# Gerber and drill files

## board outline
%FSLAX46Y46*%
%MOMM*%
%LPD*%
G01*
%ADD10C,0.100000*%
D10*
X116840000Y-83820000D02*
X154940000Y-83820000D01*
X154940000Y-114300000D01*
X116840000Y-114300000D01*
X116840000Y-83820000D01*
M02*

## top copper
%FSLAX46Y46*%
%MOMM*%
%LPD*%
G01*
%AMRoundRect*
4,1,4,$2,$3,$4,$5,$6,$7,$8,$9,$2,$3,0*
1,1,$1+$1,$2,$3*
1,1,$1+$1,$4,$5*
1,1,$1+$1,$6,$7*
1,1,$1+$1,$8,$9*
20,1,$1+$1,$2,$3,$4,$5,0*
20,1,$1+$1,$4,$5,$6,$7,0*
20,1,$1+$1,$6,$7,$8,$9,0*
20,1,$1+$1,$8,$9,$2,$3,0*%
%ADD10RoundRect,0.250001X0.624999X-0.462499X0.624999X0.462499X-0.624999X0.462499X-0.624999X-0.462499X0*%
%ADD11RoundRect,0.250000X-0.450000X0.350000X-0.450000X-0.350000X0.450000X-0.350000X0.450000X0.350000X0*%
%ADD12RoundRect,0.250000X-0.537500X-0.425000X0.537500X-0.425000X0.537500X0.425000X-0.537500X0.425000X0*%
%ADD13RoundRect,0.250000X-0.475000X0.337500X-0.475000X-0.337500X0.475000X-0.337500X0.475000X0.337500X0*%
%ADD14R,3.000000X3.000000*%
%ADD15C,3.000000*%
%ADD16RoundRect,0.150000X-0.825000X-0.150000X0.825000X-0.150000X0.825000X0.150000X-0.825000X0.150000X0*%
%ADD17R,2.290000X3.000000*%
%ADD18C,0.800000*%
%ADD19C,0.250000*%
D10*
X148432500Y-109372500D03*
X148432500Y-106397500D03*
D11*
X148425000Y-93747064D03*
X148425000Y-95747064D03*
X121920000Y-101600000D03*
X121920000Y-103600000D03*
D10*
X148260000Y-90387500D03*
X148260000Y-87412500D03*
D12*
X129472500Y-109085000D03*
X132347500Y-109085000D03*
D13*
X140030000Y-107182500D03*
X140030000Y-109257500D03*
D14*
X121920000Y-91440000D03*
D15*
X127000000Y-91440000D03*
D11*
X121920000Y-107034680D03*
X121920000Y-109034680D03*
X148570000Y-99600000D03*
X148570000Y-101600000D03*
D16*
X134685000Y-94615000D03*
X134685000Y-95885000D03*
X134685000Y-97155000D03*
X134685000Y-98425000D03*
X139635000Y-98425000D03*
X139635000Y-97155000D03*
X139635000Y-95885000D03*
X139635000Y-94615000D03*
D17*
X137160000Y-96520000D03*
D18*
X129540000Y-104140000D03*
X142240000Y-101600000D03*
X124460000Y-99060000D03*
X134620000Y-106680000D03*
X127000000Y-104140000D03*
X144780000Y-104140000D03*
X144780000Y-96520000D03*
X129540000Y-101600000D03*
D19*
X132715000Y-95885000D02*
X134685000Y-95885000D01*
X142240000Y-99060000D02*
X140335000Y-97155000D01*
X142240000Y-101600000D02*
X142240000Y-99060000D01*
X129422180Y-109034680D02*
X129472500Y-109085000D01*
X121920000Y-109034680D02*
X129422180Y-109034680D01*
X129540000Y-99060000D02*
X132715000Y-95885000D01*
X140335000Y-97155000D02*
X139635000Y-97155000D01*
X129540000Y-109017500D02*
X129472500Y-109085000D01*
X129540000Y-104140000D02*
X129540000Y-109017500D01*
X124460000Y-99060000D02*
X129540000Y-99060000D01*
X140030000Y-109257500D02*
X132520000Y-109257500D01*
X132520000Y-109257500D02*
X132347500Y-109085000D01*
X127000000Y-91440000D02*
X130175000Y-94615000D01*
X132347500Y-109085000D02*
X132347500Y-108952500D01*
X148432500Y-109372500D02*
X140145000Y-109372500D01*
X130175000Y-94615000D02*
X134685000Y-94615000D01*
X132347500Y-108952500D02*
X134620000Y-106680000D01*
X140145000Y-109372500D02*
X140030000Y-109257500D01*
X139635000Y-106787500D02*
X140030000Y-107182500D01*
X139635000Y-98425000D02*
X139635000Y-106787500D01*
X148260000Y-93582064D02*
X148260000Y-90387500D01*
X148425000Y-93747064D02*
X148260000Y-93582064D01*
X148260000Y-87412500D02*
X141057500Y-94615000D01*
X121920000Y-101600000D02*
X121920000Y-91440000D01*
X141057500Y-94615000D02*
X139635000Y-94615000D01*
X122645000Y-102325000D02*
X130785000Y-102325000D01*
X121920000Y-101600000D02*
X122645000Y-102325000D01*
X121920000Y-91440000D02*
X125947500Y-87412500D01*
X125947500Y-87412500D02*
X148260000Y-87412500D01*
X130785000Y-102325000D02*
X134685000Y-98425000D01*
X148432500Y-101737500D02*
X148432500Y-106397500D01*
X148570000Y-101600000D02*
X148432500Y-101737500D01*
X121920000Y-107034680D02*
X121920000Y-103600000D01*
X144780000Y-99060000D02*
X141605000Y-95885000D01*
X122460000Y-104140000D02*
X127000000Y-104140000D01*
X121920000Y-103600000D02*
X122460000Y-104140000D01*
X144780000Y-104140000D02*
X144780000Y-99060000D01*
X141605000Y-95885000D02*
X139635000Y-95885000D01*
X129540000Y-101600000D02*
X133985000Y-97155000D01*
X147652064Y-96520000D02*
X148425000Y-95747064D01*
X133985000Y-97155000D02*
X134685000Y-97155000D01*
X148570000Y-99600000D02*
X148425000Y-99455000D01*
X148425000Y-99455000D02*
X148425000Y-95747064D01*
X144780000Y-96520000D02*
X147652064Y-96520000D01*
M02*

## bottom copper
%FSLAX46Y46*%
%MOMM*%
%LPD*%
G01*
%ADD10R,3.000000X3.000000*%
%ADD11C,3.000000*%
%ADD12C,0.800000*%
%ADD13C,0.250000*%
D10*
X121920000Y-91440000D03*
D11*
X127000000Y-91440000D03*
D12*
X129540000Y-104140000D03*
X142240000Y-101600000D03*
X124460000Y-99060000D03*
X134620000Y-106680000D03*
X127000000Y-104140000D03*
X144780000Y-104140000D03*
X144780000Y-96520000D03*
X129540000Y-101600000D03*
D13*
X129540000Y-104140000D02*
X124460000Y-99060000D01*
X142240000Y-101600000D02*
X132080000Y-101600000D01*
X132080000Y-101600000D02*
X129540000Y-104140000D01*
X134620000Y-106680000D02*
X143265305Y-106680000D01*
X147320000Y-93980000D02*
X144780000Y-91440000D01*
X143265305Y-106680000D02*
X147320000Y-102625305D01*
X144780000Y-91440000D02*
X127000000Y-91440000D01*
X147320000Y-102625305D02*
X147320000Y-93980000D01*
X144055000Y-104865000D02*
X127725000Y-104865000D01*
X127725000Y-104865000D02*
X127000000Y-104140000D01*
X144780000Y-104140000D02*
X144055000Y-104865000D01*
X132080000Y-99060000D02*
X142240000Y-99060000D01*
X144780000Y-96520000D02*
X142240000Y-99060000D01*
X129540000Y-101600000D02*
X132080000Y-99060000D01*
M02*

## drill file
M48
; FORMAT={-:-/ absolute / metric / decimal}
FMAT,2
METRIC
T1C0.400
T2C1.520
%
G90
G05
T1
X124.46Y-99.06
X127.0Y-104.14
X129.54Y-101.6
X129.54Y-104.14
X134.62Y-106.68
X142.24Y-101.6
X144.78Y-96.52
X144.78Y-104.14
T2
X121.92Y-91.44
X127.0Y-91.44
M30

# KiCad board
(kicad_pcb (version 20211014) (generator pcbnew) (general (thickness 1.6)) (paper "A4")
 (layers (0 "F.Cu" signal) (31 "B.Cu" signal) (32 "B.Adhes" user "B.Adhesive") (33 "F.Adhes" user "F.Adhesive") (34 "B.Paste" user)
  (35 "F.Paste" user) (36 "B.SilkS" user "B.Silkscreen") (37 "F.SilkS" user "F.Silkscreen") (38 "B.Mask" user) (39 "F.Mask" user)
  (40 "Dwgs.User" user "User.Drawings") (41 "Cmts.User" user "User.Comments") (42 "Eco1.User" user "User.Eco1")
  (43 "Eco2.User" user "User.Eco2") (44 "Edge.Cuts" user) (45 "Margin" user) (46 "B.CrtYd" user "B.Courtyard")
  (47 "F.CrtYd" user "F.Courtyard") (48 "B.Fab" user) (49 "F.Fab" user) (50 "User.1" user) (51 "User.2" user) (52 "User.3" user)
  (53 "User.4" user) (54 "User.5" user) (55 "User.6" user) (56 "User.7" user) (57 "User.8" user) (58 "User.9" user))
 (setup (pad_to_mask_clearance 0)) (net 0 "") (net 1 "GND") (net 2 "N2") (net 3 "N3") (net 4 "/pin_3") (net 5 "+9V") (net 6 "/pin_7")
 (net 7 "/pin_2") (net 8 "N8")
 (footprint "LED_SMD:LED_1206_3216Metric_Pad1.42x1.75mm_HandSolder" (layer "F.Cu") (at 148.4325 107.885 90)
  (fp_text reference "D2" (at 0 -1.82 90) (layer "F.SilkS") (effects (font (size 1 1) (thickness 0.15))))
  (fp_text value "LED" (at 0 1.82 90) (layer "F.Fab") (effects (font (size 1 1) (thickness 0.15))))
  (pad "1" smd roundrect (at -1.4875 0 90) (size 1.425 1.75) (layers "F.Cu" "F.Paste" "F.Mask") (roundrect_rratio 0.175439) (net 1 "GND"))
  (pad "2" smd roundrect (at 1.4875 0 90) (size 1.425 1.75) (layers "F.Cu" "F.Paste" "F.Mask") (roundrect_rratio 0.175439) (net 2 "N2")))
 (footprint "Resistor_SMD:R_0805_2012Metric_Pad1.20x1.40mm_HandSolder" (layer "F.Cu") (at 148.425 94.747064 -90)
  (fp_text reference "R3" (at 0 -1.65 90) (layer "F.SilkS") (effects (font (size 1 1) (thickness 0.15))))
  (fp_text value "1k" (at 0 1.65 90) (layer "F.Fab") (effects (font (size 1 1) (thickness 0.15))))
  (pad "1" smd roundrect (at -1 0 270) (size 1.2 1.4) (layers "F.Cu" "F.Paste" "F.Mask") (roundrect_rratio 0.208333) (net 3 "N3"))
  (pad "2" smd roundrect (at 1 0 270) (size 1.2 1.4) (layers "F.Cu" "F.Paste" "F.Mask") (roundrect_rratio 0.208333) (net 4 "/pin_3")))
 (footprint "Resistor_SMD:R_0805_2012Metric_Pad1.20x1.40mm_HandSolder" (layer "F.Cu") (at 121.92 102.6 -90)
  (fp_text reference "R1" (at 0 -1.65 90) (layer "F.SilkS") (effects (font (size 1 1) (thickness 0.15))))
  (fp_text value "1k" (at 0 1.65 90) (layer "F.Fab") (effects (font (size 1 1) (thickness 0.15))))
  (pad "1" smd roundrect (at -1 0 270) (size 1.2 1.4) (layers "F.Cu" "F.Paste" "F.Mask") (roundrect_rratio 0.208333) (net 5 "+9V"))
  (pad "2" smd roundrect (at 1 0 270) (size 1.2 1.4) (layers "F.Cu" "F.Paste" "F.Mask") (roundrect_rratio 0.208333) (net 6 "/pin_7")))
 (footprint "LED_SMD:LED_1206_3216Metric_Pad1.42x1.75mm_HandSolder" (layer "F.Cu") (at 148.26 88.9 90)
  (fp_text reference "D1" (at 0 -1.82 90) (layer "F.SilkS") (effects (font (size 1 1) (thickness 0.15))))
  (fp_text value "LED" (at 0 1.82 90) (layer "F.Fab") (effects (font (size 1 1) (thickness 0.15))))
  (pad "1" smd roundrect (at -1.4875 0 90) (size 1.425 1.75) (layers "F.Cu" "F.Paste" "F.Mask") (roundrect_rratio 0.175439) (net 3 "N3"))
  (pad "2" smd roundrect (at 1.4875 0 90) (size 1.425 1.75) (layers "F.Cu" "F.Paste" "F.Mask") (roundrect_rratio 0.175439) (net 5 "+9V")))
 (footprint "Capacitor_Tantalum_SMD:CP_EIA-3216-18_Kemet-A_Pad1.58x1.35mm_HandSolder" (layer "F.Cu") (at 130.91 109.085)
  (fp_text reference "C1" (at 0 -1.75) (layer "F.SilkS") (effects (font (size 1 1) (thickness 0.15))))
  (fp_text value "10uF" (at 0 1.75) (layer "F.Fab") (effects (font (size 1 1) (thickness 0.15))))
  (pad "1" smd roundrect (at -1.4375 0) (size 1.575 1.35) (layers "F.Cu" "F.Paste" "F.Mask") (roundrect_rratio 0.185185) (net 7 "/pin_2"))
  (pad "2" smd roundrect (at 1.4375 0) (size 1.575 1.35) (layers "F.Cu" "F.Paste" "F.Mask") (roundrect_rratio 0.185185) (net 1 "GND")))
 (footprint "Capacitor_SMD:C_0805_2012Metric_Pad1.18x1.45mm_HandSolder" (layer "F.Cu") (at 140.03 108.22 -90)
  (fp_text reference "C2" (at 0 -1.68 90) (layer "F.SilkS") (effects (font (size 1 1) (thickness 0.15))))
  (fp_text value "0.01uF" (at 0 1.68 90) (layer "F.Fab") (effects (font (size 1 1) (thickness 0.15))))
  (pad "1" smd roundrect (at -1.0375 0 270) (size 1.175 1.45) (layers "F.Cu" "F.Paste" "F.Mask") (roundrect_rratio 0.212766) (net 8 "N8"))
  (pad "2" smd roundrect (at 1.0375 0 270) (size 1.175 1.45) (layers "F.Cu" "F.Paste" "F.Mask") (roundrect_rratio 0.212766) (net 1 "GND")))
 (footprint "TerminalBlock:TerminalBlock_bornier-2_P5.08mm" (layer "F.Cu") (at 121.92 91.44)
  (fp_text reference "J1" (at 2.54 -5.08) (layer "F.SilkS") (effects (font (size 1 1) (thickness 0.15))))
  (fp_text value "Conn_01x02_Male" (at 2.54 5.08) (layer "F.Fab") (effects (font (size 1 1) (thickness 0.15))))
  (pad "1" thru_hole rect (at 0 0) (size 3 3) (drill 1.52) (layers *.Cu *.Mask) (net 5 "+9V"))
  (pad "2" thru_hole circle (at 5.08 0) (size 3 3) (drill 1.52) (layers *.Cu *.Mask) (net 1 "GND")))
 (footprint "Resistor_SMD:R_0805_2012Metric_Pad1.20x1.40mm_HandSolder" (layer "F.Cu") (at 121.92 108.03468 -90)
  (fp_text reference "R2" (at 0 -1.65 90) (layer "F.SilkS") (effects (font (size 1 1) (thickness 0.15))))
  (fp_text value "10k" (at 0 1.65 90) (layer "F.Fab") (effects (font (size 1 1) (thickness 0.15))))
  (pad "1" smd roundrect (at -1 0 270) (size 1.2 1.4) (layers "F.Cu" "F.Paste" "F.Mask") (roundrect_rratio 0.208333) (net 6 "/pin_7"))
  (pad "2" smd roundrect (at 1 0 270) (size 1.2 1.4) (layers "F.Cu" "F.Paste" "F.Mask") (roundrect_rratio 0.208333) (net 7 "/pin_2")))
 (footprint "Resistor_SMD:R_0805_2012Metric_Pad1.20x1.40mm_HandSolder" (layer "F.Cu") (at 148.57 100.6 -90)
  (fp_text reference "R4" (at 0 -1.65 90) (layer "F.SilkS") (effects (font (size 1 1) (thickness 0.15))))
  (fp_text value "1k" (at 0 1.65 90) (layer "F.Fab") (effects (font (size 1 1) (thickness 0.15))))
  (pad "1" smd roundrect (at -1 0 270) (size 1.2 1.4) (layers "F.Cu" "F.Paste" "F.Mask") (roundrect_rratio 0.208333) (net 4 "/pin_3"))
  (pad "2" smd roundrect (at 1 0 270) (size 1.2 1.4) (layers "F.Cu" "F.Paste" "F.Mask") (roundrect_rratio 0.208333) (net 2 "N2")))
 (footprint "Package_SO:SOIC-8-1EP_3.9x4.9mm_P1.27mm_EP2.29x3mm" (layer "F.Cu") (at 137.16 96.52)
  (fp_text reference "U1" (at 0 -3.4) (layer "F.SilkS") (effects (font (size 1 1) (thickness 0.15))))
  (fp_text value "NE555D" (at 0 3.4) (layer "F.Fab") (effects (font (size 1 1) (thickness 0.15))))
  (pad "" smd roundrect (at -0.57 0.75) (size 0.92 1.21) (layers "F.Paste") (roundrect_rratio 0.25))
  (pad "" smd roundrect (at 0.57 -0.75) (size 0.92 1.21) (layers "F.Paste") (roundrect_rratio 0.25))
  (pad "" smd roundrect (at 0.57 0.75) (size 0.92 1.21) (layers "F.Paste") (roundrect_rratio 0.25))
  (pad "" smd roundrect (at -0.57 -0.75) (size 0.92 1.21) (layers "F.Paste") (roundrect_rratio 0.25))
  (pad "1" smd roundrect (at -2.475 -1.905) (size 1.95 0.6) (layers "F.Cu" "F.Paste" "F.Mask") (roundrect_rratio 0.25) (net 1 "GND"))
  (pad "2" smd roundrect (at -2.475 -0.635) (size 1.95 0.6) (layers "F.Cu" "F.Paste" "F.Mask") (roundrect_rratio 0.25) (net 7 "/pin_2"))
  (pad "3" smd roundrect (at -2.475 0.635) (size 1.95 0.6) (layers "F.Cu" "F.Paste" "F.Mask") (roundrect_rratio 0.25) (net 4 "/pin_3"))
  (pad "4" smd roundrect (at -2.475 1.905) (size 1.95 0.6) (layers "F.Cu" "F.Paste" "F.Mask") (roundrect_rratio 0.25) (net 5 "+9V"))
  (pad "5" smd roundrect (at 2.475 1.905) (size 1.95 0.6) (layers "F.Cu" "F.Paste" "F.Mask") (roundrect_rratio 0.25) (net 8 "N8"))
  (pad "6" smd roundrect (at 2.475 0.635) (size 1.95 0.6) (layers "F.Cu" "F.Paste" "F.Mask") (roundrect_rratio 0.25) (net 7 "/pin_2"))
  (pad "7" smd roundrect (at 2.475 -0.635) (size 1.95 0.6) (layers "F.Cu" "F.Paste" "F.Mask") (roundrect_rratio 0.25) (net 6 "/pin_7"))
  (pad "8" smd roundrect (at 2.475 -1.905) (size 1.95 0.6) (layers "F.Cu" "F.Paste" "F.Mask") (roundrect_rratio 0.25) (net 5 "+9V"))
  (pad "9" smd rect (at 0 0) (size 2.29 3) (layers "F.Cu" "F.Mask")))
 (gr_rect (start 116.84 83.82) (end 154.94 114.3) (layer "Edge.Cuts") (width 0.1) (fill none))
 (segment (start 132.715 95.885) (end 134.685 95.885) (width 0.25) (layer "F.Cu") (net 7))
 (segment (start 142.24 99.06) (end 140.335 97.155) (width 0.25) (layer "F.Cu") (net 7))
 (segment (start 142.24 101.6) (end 142.24 99.06) (width 0.25) (layer "F.Cu") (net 7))
 (segment (start 129.42218 109.03468) (end 129.4725 109.085) (width 0.25) (layer "F.Cu") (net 7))
 (segment (start 121.92 109.03468) (end 129.42218 109.03468) (width 0.25) (layer "F.Cu") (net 7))
 (segment (start 129.54 99.06) (end 132.715 95.885) (width 0.25) (layer "F.Cu") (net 7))
 (segment (start 140.335 97.155) (end 139.635 97.155) (width 0.25) (layer "F.Cu") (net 7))
 (segment (start 129.54 109.0175) (end 129.4725 109.085) (width 0.25) (layer "F.Cu") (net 7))
 (segment (start 129.54 104.14) (end 129.54 109.0175) (width 0.25) (layer "F.Cu") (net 7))
 (segment (start 124.46 99.06) (end 129.54 99.06) (width 0.25) (layer "F.Cu") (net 7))
 (via (at 129.54 104.14) (size 0.8) (drill 0.4) (layers "F.Cu" "B.Cu") (free) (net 7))
 (via (at 142.24 101.6) (size 0.8) (drill 0.4) (layers "F.Cu" "B.Cu") (free) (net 7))
 (via (at 124.46 99.06) (size 0.8) (drill 0.4) (layers "F.Cu" "B.Cu") (free) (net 7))
 (segment (start 129.54 104.14) (end 124.46 99.06) (width 0.25) (layer "B.Cu") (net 7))
 (segment (start 142.24 101.6) (end 132.08 101.6) (width 0.25) (layer "B.Cu") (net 7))
 (segment (start 132.08 101.6) (end 129.54 104.14) (width 0.25) (layer "B.Cu") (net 7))
 (segment (start 140.03 109.2575) (end 132.52 109.2575) (width 0.25) (layer "F.Cu") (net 1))
 (segment (start 132.52 109.2575) (end 132.3475 109.085) (width 0.25) (layer "F.Cu") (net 1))
 (segment (start 127 91.44) (end 130.175 94.615) (width 0.25) (layer "F.Cu") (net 1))
 (segment (start 132.3475 109.085) (end 132.3475 108.9525) (width 0.25) (layer "F.Cu") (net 1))
 (segment (start 148.4325 109.3725) (end 140.145 109.3725) (width 0.25) (layer "F.Cu") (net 1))
 (segment (start 130.175 94.615) (end 134.685 94.615) (width 0.25) (layer "F.Cu") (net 1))
 (segment (start 132.3475 108.9525) (end 134.62 106.68) (width 0.25) (layer "F.Cu") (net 1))
 (segment (start 140.145 109.3725) (end 140.03 109.2575) (width 0.25) (layer "F.Cu") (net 1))
 (via (at 134.62 106.68) (size 0.8) (drill 0.4) (layers "F.Cu" "B.Cu") (free) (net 1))
 (segment (start 134.62 106.68) (end 143.265305 106.68) (width 0.25) (layer "B.Cu") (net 1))
 (segment (start 147.32 93.98) (end 144.78 91.44) (width 0.25) (layer "B.Cu") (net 1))
 (segment (start 143.265305 106.68) (end 147.32 102.625305) (width 0.25) (layer "B.Cu") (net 1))
 (segment (start 144.78 91.44) (end 127 91.44) (width 0.25) (layer "B.Cu") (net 1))
 (segment (start 147.32 102.625305) (end 147.32 93.98) (width 0.25) (layer "B.Cu") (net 1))
 (segment (start 139.635 106.7875) (end 140.03 107.1825) (width 0.25) (layer "F.Cu") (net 8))
 (segment (start 139.635 98.425) (end 139.635 106.7875) (width 0.25) (layer "F.Cu") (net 8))
 (segment (start 148.26 93.582064) (end 148.26 90.3875) (width 0.25) (layer "F.Cu") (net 3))
 (segment (start 148.425 93.747064) (end 148.26 93.582064) (width 0.25) (layer "F.Cu") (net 3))
 (segment (start 148.26 87.4125) (end 141.0575 94.615) (width 0.25) (layer "F.Cu") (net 5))
 (segment (start 121.92 101.6) (end 121.92 91.44) (width 0.25) (layer "F.Cu") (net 5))
 (segment (start 141.0575 94.615) (end 139.635 94.615) (width 0.25) (layer "F.Cu") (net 5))
 (segment (start 122.645 102.325) (end 130.785 102.325) (width 0.25) (layer "F.Cu") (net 5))
 (segment (start 121.92 101.6) (end 122.645 102.325) (width 0.25) (layer "F.Cu") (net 5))
 (segment (start 121.92 91.44) (end 125.9475 87.4125) (width 0.25) (layer "F.Cu") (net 5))
 (segment (start 125.9475 87.4125) (end 148.26 87.4125) (width 0.25) (layer "F.Cu") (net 5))
 (segment (start 130.785 102.325) (end 134.685 98.425) (width 0.25) (layer "F.Cu") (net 5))
 (segment (start 148.4325 101.7375) (end 148.4325 106.3975) (width 0.25) (layer "F.Cu") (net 2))
 (segment (start 148.57 101.6) (end 148.4325 101.7375) (width 0.25) (layer "F.Cu") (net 2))
 (segment (start 121.92 107.03468) (end 121.92 103.6) (width 0.25) (layer "F.Cu") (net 6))
 (segment (start 144.78 99.06) (end 141.605 95.885) (width 0.25) (layer "F.Cu") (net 6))
 (segment (start 122.46 104.14) (end 127 104.14) (width 0.25) (layer "F.Cu") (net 6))
 (segment (start 121.92 103.6) (end 122.46 104.14) (width 0.25) (layer "F.Cu") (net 6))
 (segment (start 144.78 104.14) (end 144.78 99.06) (width 0.25) (layer "F.Cu") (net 6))
 (segment (start 141.605 95.885) (end 139.635 95.885) (width 0.25) (layer "F.Cu") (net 6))
 (via (at 127 104.14) (size 0.8) (drill 0.4) (layers "F.Cu" "B.Cu") (free) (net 6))
 (via (at 144.78 104.14) (size 0.8) (drill 0.4) (layers "F.Cu" "B.Cu") (free) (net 6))
 (segment (start 144.055 104.865) (end 127.725 104.865) (width 0.25) (layer "B.Cu") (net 6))
 (segment (start 127.725 104.865) (end 127 104.14) (width 0.25) (layer "B.Cu") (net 6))
 (segment (start 144.78 104.14) (end 144.055 104.865) (width 0.25) (layer "B.Cu") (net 6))
 (segment (start 129.54 101.6) (end 133.985 97.155) (width 0.25) (layer "F.Cu") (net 4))
 (segment (start 147.652064 96.52) (end 148.425 95.747064) (width 0.25) (layer "F.Cu") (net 4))
 (segment (start 133.985 97.155) (end 134.685 97.155) (width 0.25) (layer "F.Cu") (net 4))
 (segment (start 148.57 99.6) (end 148.425 99.455) (width 0.25) (layer "F.Cu") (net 4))
 (segment (start 148.425 99.455) (end 148.425 95.747064) (width 0.25) (layer "F.Cu") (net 4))
 (segment (start 144.78 96.52) (end 147.652064 96.52) (width 0.25) (layer "F.Cu") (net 4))
 (via (at 144.78 96.52) (size 0.8) (drill 0.4) (layers "F.Cu" "B.Cu") (free) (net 4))
 (via (at 129.54 101.6) (size 0.8) (drill 0.4) (layers "F.Cu" "B.Cu") (free) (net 4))
 (segment (start 132.08 99.06) (end 142.24 99.06) (width 0.25) (layer "B.Cu") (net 4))
 (segment (start 144.78 96.52) (end 142.24 99.06) (width 0.25) (layer "B.Cu") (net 4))
 (segment (start 129.54 101.6) (end 132.08 99.06) (width 0.25) (layer "B.Cu") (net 4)))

